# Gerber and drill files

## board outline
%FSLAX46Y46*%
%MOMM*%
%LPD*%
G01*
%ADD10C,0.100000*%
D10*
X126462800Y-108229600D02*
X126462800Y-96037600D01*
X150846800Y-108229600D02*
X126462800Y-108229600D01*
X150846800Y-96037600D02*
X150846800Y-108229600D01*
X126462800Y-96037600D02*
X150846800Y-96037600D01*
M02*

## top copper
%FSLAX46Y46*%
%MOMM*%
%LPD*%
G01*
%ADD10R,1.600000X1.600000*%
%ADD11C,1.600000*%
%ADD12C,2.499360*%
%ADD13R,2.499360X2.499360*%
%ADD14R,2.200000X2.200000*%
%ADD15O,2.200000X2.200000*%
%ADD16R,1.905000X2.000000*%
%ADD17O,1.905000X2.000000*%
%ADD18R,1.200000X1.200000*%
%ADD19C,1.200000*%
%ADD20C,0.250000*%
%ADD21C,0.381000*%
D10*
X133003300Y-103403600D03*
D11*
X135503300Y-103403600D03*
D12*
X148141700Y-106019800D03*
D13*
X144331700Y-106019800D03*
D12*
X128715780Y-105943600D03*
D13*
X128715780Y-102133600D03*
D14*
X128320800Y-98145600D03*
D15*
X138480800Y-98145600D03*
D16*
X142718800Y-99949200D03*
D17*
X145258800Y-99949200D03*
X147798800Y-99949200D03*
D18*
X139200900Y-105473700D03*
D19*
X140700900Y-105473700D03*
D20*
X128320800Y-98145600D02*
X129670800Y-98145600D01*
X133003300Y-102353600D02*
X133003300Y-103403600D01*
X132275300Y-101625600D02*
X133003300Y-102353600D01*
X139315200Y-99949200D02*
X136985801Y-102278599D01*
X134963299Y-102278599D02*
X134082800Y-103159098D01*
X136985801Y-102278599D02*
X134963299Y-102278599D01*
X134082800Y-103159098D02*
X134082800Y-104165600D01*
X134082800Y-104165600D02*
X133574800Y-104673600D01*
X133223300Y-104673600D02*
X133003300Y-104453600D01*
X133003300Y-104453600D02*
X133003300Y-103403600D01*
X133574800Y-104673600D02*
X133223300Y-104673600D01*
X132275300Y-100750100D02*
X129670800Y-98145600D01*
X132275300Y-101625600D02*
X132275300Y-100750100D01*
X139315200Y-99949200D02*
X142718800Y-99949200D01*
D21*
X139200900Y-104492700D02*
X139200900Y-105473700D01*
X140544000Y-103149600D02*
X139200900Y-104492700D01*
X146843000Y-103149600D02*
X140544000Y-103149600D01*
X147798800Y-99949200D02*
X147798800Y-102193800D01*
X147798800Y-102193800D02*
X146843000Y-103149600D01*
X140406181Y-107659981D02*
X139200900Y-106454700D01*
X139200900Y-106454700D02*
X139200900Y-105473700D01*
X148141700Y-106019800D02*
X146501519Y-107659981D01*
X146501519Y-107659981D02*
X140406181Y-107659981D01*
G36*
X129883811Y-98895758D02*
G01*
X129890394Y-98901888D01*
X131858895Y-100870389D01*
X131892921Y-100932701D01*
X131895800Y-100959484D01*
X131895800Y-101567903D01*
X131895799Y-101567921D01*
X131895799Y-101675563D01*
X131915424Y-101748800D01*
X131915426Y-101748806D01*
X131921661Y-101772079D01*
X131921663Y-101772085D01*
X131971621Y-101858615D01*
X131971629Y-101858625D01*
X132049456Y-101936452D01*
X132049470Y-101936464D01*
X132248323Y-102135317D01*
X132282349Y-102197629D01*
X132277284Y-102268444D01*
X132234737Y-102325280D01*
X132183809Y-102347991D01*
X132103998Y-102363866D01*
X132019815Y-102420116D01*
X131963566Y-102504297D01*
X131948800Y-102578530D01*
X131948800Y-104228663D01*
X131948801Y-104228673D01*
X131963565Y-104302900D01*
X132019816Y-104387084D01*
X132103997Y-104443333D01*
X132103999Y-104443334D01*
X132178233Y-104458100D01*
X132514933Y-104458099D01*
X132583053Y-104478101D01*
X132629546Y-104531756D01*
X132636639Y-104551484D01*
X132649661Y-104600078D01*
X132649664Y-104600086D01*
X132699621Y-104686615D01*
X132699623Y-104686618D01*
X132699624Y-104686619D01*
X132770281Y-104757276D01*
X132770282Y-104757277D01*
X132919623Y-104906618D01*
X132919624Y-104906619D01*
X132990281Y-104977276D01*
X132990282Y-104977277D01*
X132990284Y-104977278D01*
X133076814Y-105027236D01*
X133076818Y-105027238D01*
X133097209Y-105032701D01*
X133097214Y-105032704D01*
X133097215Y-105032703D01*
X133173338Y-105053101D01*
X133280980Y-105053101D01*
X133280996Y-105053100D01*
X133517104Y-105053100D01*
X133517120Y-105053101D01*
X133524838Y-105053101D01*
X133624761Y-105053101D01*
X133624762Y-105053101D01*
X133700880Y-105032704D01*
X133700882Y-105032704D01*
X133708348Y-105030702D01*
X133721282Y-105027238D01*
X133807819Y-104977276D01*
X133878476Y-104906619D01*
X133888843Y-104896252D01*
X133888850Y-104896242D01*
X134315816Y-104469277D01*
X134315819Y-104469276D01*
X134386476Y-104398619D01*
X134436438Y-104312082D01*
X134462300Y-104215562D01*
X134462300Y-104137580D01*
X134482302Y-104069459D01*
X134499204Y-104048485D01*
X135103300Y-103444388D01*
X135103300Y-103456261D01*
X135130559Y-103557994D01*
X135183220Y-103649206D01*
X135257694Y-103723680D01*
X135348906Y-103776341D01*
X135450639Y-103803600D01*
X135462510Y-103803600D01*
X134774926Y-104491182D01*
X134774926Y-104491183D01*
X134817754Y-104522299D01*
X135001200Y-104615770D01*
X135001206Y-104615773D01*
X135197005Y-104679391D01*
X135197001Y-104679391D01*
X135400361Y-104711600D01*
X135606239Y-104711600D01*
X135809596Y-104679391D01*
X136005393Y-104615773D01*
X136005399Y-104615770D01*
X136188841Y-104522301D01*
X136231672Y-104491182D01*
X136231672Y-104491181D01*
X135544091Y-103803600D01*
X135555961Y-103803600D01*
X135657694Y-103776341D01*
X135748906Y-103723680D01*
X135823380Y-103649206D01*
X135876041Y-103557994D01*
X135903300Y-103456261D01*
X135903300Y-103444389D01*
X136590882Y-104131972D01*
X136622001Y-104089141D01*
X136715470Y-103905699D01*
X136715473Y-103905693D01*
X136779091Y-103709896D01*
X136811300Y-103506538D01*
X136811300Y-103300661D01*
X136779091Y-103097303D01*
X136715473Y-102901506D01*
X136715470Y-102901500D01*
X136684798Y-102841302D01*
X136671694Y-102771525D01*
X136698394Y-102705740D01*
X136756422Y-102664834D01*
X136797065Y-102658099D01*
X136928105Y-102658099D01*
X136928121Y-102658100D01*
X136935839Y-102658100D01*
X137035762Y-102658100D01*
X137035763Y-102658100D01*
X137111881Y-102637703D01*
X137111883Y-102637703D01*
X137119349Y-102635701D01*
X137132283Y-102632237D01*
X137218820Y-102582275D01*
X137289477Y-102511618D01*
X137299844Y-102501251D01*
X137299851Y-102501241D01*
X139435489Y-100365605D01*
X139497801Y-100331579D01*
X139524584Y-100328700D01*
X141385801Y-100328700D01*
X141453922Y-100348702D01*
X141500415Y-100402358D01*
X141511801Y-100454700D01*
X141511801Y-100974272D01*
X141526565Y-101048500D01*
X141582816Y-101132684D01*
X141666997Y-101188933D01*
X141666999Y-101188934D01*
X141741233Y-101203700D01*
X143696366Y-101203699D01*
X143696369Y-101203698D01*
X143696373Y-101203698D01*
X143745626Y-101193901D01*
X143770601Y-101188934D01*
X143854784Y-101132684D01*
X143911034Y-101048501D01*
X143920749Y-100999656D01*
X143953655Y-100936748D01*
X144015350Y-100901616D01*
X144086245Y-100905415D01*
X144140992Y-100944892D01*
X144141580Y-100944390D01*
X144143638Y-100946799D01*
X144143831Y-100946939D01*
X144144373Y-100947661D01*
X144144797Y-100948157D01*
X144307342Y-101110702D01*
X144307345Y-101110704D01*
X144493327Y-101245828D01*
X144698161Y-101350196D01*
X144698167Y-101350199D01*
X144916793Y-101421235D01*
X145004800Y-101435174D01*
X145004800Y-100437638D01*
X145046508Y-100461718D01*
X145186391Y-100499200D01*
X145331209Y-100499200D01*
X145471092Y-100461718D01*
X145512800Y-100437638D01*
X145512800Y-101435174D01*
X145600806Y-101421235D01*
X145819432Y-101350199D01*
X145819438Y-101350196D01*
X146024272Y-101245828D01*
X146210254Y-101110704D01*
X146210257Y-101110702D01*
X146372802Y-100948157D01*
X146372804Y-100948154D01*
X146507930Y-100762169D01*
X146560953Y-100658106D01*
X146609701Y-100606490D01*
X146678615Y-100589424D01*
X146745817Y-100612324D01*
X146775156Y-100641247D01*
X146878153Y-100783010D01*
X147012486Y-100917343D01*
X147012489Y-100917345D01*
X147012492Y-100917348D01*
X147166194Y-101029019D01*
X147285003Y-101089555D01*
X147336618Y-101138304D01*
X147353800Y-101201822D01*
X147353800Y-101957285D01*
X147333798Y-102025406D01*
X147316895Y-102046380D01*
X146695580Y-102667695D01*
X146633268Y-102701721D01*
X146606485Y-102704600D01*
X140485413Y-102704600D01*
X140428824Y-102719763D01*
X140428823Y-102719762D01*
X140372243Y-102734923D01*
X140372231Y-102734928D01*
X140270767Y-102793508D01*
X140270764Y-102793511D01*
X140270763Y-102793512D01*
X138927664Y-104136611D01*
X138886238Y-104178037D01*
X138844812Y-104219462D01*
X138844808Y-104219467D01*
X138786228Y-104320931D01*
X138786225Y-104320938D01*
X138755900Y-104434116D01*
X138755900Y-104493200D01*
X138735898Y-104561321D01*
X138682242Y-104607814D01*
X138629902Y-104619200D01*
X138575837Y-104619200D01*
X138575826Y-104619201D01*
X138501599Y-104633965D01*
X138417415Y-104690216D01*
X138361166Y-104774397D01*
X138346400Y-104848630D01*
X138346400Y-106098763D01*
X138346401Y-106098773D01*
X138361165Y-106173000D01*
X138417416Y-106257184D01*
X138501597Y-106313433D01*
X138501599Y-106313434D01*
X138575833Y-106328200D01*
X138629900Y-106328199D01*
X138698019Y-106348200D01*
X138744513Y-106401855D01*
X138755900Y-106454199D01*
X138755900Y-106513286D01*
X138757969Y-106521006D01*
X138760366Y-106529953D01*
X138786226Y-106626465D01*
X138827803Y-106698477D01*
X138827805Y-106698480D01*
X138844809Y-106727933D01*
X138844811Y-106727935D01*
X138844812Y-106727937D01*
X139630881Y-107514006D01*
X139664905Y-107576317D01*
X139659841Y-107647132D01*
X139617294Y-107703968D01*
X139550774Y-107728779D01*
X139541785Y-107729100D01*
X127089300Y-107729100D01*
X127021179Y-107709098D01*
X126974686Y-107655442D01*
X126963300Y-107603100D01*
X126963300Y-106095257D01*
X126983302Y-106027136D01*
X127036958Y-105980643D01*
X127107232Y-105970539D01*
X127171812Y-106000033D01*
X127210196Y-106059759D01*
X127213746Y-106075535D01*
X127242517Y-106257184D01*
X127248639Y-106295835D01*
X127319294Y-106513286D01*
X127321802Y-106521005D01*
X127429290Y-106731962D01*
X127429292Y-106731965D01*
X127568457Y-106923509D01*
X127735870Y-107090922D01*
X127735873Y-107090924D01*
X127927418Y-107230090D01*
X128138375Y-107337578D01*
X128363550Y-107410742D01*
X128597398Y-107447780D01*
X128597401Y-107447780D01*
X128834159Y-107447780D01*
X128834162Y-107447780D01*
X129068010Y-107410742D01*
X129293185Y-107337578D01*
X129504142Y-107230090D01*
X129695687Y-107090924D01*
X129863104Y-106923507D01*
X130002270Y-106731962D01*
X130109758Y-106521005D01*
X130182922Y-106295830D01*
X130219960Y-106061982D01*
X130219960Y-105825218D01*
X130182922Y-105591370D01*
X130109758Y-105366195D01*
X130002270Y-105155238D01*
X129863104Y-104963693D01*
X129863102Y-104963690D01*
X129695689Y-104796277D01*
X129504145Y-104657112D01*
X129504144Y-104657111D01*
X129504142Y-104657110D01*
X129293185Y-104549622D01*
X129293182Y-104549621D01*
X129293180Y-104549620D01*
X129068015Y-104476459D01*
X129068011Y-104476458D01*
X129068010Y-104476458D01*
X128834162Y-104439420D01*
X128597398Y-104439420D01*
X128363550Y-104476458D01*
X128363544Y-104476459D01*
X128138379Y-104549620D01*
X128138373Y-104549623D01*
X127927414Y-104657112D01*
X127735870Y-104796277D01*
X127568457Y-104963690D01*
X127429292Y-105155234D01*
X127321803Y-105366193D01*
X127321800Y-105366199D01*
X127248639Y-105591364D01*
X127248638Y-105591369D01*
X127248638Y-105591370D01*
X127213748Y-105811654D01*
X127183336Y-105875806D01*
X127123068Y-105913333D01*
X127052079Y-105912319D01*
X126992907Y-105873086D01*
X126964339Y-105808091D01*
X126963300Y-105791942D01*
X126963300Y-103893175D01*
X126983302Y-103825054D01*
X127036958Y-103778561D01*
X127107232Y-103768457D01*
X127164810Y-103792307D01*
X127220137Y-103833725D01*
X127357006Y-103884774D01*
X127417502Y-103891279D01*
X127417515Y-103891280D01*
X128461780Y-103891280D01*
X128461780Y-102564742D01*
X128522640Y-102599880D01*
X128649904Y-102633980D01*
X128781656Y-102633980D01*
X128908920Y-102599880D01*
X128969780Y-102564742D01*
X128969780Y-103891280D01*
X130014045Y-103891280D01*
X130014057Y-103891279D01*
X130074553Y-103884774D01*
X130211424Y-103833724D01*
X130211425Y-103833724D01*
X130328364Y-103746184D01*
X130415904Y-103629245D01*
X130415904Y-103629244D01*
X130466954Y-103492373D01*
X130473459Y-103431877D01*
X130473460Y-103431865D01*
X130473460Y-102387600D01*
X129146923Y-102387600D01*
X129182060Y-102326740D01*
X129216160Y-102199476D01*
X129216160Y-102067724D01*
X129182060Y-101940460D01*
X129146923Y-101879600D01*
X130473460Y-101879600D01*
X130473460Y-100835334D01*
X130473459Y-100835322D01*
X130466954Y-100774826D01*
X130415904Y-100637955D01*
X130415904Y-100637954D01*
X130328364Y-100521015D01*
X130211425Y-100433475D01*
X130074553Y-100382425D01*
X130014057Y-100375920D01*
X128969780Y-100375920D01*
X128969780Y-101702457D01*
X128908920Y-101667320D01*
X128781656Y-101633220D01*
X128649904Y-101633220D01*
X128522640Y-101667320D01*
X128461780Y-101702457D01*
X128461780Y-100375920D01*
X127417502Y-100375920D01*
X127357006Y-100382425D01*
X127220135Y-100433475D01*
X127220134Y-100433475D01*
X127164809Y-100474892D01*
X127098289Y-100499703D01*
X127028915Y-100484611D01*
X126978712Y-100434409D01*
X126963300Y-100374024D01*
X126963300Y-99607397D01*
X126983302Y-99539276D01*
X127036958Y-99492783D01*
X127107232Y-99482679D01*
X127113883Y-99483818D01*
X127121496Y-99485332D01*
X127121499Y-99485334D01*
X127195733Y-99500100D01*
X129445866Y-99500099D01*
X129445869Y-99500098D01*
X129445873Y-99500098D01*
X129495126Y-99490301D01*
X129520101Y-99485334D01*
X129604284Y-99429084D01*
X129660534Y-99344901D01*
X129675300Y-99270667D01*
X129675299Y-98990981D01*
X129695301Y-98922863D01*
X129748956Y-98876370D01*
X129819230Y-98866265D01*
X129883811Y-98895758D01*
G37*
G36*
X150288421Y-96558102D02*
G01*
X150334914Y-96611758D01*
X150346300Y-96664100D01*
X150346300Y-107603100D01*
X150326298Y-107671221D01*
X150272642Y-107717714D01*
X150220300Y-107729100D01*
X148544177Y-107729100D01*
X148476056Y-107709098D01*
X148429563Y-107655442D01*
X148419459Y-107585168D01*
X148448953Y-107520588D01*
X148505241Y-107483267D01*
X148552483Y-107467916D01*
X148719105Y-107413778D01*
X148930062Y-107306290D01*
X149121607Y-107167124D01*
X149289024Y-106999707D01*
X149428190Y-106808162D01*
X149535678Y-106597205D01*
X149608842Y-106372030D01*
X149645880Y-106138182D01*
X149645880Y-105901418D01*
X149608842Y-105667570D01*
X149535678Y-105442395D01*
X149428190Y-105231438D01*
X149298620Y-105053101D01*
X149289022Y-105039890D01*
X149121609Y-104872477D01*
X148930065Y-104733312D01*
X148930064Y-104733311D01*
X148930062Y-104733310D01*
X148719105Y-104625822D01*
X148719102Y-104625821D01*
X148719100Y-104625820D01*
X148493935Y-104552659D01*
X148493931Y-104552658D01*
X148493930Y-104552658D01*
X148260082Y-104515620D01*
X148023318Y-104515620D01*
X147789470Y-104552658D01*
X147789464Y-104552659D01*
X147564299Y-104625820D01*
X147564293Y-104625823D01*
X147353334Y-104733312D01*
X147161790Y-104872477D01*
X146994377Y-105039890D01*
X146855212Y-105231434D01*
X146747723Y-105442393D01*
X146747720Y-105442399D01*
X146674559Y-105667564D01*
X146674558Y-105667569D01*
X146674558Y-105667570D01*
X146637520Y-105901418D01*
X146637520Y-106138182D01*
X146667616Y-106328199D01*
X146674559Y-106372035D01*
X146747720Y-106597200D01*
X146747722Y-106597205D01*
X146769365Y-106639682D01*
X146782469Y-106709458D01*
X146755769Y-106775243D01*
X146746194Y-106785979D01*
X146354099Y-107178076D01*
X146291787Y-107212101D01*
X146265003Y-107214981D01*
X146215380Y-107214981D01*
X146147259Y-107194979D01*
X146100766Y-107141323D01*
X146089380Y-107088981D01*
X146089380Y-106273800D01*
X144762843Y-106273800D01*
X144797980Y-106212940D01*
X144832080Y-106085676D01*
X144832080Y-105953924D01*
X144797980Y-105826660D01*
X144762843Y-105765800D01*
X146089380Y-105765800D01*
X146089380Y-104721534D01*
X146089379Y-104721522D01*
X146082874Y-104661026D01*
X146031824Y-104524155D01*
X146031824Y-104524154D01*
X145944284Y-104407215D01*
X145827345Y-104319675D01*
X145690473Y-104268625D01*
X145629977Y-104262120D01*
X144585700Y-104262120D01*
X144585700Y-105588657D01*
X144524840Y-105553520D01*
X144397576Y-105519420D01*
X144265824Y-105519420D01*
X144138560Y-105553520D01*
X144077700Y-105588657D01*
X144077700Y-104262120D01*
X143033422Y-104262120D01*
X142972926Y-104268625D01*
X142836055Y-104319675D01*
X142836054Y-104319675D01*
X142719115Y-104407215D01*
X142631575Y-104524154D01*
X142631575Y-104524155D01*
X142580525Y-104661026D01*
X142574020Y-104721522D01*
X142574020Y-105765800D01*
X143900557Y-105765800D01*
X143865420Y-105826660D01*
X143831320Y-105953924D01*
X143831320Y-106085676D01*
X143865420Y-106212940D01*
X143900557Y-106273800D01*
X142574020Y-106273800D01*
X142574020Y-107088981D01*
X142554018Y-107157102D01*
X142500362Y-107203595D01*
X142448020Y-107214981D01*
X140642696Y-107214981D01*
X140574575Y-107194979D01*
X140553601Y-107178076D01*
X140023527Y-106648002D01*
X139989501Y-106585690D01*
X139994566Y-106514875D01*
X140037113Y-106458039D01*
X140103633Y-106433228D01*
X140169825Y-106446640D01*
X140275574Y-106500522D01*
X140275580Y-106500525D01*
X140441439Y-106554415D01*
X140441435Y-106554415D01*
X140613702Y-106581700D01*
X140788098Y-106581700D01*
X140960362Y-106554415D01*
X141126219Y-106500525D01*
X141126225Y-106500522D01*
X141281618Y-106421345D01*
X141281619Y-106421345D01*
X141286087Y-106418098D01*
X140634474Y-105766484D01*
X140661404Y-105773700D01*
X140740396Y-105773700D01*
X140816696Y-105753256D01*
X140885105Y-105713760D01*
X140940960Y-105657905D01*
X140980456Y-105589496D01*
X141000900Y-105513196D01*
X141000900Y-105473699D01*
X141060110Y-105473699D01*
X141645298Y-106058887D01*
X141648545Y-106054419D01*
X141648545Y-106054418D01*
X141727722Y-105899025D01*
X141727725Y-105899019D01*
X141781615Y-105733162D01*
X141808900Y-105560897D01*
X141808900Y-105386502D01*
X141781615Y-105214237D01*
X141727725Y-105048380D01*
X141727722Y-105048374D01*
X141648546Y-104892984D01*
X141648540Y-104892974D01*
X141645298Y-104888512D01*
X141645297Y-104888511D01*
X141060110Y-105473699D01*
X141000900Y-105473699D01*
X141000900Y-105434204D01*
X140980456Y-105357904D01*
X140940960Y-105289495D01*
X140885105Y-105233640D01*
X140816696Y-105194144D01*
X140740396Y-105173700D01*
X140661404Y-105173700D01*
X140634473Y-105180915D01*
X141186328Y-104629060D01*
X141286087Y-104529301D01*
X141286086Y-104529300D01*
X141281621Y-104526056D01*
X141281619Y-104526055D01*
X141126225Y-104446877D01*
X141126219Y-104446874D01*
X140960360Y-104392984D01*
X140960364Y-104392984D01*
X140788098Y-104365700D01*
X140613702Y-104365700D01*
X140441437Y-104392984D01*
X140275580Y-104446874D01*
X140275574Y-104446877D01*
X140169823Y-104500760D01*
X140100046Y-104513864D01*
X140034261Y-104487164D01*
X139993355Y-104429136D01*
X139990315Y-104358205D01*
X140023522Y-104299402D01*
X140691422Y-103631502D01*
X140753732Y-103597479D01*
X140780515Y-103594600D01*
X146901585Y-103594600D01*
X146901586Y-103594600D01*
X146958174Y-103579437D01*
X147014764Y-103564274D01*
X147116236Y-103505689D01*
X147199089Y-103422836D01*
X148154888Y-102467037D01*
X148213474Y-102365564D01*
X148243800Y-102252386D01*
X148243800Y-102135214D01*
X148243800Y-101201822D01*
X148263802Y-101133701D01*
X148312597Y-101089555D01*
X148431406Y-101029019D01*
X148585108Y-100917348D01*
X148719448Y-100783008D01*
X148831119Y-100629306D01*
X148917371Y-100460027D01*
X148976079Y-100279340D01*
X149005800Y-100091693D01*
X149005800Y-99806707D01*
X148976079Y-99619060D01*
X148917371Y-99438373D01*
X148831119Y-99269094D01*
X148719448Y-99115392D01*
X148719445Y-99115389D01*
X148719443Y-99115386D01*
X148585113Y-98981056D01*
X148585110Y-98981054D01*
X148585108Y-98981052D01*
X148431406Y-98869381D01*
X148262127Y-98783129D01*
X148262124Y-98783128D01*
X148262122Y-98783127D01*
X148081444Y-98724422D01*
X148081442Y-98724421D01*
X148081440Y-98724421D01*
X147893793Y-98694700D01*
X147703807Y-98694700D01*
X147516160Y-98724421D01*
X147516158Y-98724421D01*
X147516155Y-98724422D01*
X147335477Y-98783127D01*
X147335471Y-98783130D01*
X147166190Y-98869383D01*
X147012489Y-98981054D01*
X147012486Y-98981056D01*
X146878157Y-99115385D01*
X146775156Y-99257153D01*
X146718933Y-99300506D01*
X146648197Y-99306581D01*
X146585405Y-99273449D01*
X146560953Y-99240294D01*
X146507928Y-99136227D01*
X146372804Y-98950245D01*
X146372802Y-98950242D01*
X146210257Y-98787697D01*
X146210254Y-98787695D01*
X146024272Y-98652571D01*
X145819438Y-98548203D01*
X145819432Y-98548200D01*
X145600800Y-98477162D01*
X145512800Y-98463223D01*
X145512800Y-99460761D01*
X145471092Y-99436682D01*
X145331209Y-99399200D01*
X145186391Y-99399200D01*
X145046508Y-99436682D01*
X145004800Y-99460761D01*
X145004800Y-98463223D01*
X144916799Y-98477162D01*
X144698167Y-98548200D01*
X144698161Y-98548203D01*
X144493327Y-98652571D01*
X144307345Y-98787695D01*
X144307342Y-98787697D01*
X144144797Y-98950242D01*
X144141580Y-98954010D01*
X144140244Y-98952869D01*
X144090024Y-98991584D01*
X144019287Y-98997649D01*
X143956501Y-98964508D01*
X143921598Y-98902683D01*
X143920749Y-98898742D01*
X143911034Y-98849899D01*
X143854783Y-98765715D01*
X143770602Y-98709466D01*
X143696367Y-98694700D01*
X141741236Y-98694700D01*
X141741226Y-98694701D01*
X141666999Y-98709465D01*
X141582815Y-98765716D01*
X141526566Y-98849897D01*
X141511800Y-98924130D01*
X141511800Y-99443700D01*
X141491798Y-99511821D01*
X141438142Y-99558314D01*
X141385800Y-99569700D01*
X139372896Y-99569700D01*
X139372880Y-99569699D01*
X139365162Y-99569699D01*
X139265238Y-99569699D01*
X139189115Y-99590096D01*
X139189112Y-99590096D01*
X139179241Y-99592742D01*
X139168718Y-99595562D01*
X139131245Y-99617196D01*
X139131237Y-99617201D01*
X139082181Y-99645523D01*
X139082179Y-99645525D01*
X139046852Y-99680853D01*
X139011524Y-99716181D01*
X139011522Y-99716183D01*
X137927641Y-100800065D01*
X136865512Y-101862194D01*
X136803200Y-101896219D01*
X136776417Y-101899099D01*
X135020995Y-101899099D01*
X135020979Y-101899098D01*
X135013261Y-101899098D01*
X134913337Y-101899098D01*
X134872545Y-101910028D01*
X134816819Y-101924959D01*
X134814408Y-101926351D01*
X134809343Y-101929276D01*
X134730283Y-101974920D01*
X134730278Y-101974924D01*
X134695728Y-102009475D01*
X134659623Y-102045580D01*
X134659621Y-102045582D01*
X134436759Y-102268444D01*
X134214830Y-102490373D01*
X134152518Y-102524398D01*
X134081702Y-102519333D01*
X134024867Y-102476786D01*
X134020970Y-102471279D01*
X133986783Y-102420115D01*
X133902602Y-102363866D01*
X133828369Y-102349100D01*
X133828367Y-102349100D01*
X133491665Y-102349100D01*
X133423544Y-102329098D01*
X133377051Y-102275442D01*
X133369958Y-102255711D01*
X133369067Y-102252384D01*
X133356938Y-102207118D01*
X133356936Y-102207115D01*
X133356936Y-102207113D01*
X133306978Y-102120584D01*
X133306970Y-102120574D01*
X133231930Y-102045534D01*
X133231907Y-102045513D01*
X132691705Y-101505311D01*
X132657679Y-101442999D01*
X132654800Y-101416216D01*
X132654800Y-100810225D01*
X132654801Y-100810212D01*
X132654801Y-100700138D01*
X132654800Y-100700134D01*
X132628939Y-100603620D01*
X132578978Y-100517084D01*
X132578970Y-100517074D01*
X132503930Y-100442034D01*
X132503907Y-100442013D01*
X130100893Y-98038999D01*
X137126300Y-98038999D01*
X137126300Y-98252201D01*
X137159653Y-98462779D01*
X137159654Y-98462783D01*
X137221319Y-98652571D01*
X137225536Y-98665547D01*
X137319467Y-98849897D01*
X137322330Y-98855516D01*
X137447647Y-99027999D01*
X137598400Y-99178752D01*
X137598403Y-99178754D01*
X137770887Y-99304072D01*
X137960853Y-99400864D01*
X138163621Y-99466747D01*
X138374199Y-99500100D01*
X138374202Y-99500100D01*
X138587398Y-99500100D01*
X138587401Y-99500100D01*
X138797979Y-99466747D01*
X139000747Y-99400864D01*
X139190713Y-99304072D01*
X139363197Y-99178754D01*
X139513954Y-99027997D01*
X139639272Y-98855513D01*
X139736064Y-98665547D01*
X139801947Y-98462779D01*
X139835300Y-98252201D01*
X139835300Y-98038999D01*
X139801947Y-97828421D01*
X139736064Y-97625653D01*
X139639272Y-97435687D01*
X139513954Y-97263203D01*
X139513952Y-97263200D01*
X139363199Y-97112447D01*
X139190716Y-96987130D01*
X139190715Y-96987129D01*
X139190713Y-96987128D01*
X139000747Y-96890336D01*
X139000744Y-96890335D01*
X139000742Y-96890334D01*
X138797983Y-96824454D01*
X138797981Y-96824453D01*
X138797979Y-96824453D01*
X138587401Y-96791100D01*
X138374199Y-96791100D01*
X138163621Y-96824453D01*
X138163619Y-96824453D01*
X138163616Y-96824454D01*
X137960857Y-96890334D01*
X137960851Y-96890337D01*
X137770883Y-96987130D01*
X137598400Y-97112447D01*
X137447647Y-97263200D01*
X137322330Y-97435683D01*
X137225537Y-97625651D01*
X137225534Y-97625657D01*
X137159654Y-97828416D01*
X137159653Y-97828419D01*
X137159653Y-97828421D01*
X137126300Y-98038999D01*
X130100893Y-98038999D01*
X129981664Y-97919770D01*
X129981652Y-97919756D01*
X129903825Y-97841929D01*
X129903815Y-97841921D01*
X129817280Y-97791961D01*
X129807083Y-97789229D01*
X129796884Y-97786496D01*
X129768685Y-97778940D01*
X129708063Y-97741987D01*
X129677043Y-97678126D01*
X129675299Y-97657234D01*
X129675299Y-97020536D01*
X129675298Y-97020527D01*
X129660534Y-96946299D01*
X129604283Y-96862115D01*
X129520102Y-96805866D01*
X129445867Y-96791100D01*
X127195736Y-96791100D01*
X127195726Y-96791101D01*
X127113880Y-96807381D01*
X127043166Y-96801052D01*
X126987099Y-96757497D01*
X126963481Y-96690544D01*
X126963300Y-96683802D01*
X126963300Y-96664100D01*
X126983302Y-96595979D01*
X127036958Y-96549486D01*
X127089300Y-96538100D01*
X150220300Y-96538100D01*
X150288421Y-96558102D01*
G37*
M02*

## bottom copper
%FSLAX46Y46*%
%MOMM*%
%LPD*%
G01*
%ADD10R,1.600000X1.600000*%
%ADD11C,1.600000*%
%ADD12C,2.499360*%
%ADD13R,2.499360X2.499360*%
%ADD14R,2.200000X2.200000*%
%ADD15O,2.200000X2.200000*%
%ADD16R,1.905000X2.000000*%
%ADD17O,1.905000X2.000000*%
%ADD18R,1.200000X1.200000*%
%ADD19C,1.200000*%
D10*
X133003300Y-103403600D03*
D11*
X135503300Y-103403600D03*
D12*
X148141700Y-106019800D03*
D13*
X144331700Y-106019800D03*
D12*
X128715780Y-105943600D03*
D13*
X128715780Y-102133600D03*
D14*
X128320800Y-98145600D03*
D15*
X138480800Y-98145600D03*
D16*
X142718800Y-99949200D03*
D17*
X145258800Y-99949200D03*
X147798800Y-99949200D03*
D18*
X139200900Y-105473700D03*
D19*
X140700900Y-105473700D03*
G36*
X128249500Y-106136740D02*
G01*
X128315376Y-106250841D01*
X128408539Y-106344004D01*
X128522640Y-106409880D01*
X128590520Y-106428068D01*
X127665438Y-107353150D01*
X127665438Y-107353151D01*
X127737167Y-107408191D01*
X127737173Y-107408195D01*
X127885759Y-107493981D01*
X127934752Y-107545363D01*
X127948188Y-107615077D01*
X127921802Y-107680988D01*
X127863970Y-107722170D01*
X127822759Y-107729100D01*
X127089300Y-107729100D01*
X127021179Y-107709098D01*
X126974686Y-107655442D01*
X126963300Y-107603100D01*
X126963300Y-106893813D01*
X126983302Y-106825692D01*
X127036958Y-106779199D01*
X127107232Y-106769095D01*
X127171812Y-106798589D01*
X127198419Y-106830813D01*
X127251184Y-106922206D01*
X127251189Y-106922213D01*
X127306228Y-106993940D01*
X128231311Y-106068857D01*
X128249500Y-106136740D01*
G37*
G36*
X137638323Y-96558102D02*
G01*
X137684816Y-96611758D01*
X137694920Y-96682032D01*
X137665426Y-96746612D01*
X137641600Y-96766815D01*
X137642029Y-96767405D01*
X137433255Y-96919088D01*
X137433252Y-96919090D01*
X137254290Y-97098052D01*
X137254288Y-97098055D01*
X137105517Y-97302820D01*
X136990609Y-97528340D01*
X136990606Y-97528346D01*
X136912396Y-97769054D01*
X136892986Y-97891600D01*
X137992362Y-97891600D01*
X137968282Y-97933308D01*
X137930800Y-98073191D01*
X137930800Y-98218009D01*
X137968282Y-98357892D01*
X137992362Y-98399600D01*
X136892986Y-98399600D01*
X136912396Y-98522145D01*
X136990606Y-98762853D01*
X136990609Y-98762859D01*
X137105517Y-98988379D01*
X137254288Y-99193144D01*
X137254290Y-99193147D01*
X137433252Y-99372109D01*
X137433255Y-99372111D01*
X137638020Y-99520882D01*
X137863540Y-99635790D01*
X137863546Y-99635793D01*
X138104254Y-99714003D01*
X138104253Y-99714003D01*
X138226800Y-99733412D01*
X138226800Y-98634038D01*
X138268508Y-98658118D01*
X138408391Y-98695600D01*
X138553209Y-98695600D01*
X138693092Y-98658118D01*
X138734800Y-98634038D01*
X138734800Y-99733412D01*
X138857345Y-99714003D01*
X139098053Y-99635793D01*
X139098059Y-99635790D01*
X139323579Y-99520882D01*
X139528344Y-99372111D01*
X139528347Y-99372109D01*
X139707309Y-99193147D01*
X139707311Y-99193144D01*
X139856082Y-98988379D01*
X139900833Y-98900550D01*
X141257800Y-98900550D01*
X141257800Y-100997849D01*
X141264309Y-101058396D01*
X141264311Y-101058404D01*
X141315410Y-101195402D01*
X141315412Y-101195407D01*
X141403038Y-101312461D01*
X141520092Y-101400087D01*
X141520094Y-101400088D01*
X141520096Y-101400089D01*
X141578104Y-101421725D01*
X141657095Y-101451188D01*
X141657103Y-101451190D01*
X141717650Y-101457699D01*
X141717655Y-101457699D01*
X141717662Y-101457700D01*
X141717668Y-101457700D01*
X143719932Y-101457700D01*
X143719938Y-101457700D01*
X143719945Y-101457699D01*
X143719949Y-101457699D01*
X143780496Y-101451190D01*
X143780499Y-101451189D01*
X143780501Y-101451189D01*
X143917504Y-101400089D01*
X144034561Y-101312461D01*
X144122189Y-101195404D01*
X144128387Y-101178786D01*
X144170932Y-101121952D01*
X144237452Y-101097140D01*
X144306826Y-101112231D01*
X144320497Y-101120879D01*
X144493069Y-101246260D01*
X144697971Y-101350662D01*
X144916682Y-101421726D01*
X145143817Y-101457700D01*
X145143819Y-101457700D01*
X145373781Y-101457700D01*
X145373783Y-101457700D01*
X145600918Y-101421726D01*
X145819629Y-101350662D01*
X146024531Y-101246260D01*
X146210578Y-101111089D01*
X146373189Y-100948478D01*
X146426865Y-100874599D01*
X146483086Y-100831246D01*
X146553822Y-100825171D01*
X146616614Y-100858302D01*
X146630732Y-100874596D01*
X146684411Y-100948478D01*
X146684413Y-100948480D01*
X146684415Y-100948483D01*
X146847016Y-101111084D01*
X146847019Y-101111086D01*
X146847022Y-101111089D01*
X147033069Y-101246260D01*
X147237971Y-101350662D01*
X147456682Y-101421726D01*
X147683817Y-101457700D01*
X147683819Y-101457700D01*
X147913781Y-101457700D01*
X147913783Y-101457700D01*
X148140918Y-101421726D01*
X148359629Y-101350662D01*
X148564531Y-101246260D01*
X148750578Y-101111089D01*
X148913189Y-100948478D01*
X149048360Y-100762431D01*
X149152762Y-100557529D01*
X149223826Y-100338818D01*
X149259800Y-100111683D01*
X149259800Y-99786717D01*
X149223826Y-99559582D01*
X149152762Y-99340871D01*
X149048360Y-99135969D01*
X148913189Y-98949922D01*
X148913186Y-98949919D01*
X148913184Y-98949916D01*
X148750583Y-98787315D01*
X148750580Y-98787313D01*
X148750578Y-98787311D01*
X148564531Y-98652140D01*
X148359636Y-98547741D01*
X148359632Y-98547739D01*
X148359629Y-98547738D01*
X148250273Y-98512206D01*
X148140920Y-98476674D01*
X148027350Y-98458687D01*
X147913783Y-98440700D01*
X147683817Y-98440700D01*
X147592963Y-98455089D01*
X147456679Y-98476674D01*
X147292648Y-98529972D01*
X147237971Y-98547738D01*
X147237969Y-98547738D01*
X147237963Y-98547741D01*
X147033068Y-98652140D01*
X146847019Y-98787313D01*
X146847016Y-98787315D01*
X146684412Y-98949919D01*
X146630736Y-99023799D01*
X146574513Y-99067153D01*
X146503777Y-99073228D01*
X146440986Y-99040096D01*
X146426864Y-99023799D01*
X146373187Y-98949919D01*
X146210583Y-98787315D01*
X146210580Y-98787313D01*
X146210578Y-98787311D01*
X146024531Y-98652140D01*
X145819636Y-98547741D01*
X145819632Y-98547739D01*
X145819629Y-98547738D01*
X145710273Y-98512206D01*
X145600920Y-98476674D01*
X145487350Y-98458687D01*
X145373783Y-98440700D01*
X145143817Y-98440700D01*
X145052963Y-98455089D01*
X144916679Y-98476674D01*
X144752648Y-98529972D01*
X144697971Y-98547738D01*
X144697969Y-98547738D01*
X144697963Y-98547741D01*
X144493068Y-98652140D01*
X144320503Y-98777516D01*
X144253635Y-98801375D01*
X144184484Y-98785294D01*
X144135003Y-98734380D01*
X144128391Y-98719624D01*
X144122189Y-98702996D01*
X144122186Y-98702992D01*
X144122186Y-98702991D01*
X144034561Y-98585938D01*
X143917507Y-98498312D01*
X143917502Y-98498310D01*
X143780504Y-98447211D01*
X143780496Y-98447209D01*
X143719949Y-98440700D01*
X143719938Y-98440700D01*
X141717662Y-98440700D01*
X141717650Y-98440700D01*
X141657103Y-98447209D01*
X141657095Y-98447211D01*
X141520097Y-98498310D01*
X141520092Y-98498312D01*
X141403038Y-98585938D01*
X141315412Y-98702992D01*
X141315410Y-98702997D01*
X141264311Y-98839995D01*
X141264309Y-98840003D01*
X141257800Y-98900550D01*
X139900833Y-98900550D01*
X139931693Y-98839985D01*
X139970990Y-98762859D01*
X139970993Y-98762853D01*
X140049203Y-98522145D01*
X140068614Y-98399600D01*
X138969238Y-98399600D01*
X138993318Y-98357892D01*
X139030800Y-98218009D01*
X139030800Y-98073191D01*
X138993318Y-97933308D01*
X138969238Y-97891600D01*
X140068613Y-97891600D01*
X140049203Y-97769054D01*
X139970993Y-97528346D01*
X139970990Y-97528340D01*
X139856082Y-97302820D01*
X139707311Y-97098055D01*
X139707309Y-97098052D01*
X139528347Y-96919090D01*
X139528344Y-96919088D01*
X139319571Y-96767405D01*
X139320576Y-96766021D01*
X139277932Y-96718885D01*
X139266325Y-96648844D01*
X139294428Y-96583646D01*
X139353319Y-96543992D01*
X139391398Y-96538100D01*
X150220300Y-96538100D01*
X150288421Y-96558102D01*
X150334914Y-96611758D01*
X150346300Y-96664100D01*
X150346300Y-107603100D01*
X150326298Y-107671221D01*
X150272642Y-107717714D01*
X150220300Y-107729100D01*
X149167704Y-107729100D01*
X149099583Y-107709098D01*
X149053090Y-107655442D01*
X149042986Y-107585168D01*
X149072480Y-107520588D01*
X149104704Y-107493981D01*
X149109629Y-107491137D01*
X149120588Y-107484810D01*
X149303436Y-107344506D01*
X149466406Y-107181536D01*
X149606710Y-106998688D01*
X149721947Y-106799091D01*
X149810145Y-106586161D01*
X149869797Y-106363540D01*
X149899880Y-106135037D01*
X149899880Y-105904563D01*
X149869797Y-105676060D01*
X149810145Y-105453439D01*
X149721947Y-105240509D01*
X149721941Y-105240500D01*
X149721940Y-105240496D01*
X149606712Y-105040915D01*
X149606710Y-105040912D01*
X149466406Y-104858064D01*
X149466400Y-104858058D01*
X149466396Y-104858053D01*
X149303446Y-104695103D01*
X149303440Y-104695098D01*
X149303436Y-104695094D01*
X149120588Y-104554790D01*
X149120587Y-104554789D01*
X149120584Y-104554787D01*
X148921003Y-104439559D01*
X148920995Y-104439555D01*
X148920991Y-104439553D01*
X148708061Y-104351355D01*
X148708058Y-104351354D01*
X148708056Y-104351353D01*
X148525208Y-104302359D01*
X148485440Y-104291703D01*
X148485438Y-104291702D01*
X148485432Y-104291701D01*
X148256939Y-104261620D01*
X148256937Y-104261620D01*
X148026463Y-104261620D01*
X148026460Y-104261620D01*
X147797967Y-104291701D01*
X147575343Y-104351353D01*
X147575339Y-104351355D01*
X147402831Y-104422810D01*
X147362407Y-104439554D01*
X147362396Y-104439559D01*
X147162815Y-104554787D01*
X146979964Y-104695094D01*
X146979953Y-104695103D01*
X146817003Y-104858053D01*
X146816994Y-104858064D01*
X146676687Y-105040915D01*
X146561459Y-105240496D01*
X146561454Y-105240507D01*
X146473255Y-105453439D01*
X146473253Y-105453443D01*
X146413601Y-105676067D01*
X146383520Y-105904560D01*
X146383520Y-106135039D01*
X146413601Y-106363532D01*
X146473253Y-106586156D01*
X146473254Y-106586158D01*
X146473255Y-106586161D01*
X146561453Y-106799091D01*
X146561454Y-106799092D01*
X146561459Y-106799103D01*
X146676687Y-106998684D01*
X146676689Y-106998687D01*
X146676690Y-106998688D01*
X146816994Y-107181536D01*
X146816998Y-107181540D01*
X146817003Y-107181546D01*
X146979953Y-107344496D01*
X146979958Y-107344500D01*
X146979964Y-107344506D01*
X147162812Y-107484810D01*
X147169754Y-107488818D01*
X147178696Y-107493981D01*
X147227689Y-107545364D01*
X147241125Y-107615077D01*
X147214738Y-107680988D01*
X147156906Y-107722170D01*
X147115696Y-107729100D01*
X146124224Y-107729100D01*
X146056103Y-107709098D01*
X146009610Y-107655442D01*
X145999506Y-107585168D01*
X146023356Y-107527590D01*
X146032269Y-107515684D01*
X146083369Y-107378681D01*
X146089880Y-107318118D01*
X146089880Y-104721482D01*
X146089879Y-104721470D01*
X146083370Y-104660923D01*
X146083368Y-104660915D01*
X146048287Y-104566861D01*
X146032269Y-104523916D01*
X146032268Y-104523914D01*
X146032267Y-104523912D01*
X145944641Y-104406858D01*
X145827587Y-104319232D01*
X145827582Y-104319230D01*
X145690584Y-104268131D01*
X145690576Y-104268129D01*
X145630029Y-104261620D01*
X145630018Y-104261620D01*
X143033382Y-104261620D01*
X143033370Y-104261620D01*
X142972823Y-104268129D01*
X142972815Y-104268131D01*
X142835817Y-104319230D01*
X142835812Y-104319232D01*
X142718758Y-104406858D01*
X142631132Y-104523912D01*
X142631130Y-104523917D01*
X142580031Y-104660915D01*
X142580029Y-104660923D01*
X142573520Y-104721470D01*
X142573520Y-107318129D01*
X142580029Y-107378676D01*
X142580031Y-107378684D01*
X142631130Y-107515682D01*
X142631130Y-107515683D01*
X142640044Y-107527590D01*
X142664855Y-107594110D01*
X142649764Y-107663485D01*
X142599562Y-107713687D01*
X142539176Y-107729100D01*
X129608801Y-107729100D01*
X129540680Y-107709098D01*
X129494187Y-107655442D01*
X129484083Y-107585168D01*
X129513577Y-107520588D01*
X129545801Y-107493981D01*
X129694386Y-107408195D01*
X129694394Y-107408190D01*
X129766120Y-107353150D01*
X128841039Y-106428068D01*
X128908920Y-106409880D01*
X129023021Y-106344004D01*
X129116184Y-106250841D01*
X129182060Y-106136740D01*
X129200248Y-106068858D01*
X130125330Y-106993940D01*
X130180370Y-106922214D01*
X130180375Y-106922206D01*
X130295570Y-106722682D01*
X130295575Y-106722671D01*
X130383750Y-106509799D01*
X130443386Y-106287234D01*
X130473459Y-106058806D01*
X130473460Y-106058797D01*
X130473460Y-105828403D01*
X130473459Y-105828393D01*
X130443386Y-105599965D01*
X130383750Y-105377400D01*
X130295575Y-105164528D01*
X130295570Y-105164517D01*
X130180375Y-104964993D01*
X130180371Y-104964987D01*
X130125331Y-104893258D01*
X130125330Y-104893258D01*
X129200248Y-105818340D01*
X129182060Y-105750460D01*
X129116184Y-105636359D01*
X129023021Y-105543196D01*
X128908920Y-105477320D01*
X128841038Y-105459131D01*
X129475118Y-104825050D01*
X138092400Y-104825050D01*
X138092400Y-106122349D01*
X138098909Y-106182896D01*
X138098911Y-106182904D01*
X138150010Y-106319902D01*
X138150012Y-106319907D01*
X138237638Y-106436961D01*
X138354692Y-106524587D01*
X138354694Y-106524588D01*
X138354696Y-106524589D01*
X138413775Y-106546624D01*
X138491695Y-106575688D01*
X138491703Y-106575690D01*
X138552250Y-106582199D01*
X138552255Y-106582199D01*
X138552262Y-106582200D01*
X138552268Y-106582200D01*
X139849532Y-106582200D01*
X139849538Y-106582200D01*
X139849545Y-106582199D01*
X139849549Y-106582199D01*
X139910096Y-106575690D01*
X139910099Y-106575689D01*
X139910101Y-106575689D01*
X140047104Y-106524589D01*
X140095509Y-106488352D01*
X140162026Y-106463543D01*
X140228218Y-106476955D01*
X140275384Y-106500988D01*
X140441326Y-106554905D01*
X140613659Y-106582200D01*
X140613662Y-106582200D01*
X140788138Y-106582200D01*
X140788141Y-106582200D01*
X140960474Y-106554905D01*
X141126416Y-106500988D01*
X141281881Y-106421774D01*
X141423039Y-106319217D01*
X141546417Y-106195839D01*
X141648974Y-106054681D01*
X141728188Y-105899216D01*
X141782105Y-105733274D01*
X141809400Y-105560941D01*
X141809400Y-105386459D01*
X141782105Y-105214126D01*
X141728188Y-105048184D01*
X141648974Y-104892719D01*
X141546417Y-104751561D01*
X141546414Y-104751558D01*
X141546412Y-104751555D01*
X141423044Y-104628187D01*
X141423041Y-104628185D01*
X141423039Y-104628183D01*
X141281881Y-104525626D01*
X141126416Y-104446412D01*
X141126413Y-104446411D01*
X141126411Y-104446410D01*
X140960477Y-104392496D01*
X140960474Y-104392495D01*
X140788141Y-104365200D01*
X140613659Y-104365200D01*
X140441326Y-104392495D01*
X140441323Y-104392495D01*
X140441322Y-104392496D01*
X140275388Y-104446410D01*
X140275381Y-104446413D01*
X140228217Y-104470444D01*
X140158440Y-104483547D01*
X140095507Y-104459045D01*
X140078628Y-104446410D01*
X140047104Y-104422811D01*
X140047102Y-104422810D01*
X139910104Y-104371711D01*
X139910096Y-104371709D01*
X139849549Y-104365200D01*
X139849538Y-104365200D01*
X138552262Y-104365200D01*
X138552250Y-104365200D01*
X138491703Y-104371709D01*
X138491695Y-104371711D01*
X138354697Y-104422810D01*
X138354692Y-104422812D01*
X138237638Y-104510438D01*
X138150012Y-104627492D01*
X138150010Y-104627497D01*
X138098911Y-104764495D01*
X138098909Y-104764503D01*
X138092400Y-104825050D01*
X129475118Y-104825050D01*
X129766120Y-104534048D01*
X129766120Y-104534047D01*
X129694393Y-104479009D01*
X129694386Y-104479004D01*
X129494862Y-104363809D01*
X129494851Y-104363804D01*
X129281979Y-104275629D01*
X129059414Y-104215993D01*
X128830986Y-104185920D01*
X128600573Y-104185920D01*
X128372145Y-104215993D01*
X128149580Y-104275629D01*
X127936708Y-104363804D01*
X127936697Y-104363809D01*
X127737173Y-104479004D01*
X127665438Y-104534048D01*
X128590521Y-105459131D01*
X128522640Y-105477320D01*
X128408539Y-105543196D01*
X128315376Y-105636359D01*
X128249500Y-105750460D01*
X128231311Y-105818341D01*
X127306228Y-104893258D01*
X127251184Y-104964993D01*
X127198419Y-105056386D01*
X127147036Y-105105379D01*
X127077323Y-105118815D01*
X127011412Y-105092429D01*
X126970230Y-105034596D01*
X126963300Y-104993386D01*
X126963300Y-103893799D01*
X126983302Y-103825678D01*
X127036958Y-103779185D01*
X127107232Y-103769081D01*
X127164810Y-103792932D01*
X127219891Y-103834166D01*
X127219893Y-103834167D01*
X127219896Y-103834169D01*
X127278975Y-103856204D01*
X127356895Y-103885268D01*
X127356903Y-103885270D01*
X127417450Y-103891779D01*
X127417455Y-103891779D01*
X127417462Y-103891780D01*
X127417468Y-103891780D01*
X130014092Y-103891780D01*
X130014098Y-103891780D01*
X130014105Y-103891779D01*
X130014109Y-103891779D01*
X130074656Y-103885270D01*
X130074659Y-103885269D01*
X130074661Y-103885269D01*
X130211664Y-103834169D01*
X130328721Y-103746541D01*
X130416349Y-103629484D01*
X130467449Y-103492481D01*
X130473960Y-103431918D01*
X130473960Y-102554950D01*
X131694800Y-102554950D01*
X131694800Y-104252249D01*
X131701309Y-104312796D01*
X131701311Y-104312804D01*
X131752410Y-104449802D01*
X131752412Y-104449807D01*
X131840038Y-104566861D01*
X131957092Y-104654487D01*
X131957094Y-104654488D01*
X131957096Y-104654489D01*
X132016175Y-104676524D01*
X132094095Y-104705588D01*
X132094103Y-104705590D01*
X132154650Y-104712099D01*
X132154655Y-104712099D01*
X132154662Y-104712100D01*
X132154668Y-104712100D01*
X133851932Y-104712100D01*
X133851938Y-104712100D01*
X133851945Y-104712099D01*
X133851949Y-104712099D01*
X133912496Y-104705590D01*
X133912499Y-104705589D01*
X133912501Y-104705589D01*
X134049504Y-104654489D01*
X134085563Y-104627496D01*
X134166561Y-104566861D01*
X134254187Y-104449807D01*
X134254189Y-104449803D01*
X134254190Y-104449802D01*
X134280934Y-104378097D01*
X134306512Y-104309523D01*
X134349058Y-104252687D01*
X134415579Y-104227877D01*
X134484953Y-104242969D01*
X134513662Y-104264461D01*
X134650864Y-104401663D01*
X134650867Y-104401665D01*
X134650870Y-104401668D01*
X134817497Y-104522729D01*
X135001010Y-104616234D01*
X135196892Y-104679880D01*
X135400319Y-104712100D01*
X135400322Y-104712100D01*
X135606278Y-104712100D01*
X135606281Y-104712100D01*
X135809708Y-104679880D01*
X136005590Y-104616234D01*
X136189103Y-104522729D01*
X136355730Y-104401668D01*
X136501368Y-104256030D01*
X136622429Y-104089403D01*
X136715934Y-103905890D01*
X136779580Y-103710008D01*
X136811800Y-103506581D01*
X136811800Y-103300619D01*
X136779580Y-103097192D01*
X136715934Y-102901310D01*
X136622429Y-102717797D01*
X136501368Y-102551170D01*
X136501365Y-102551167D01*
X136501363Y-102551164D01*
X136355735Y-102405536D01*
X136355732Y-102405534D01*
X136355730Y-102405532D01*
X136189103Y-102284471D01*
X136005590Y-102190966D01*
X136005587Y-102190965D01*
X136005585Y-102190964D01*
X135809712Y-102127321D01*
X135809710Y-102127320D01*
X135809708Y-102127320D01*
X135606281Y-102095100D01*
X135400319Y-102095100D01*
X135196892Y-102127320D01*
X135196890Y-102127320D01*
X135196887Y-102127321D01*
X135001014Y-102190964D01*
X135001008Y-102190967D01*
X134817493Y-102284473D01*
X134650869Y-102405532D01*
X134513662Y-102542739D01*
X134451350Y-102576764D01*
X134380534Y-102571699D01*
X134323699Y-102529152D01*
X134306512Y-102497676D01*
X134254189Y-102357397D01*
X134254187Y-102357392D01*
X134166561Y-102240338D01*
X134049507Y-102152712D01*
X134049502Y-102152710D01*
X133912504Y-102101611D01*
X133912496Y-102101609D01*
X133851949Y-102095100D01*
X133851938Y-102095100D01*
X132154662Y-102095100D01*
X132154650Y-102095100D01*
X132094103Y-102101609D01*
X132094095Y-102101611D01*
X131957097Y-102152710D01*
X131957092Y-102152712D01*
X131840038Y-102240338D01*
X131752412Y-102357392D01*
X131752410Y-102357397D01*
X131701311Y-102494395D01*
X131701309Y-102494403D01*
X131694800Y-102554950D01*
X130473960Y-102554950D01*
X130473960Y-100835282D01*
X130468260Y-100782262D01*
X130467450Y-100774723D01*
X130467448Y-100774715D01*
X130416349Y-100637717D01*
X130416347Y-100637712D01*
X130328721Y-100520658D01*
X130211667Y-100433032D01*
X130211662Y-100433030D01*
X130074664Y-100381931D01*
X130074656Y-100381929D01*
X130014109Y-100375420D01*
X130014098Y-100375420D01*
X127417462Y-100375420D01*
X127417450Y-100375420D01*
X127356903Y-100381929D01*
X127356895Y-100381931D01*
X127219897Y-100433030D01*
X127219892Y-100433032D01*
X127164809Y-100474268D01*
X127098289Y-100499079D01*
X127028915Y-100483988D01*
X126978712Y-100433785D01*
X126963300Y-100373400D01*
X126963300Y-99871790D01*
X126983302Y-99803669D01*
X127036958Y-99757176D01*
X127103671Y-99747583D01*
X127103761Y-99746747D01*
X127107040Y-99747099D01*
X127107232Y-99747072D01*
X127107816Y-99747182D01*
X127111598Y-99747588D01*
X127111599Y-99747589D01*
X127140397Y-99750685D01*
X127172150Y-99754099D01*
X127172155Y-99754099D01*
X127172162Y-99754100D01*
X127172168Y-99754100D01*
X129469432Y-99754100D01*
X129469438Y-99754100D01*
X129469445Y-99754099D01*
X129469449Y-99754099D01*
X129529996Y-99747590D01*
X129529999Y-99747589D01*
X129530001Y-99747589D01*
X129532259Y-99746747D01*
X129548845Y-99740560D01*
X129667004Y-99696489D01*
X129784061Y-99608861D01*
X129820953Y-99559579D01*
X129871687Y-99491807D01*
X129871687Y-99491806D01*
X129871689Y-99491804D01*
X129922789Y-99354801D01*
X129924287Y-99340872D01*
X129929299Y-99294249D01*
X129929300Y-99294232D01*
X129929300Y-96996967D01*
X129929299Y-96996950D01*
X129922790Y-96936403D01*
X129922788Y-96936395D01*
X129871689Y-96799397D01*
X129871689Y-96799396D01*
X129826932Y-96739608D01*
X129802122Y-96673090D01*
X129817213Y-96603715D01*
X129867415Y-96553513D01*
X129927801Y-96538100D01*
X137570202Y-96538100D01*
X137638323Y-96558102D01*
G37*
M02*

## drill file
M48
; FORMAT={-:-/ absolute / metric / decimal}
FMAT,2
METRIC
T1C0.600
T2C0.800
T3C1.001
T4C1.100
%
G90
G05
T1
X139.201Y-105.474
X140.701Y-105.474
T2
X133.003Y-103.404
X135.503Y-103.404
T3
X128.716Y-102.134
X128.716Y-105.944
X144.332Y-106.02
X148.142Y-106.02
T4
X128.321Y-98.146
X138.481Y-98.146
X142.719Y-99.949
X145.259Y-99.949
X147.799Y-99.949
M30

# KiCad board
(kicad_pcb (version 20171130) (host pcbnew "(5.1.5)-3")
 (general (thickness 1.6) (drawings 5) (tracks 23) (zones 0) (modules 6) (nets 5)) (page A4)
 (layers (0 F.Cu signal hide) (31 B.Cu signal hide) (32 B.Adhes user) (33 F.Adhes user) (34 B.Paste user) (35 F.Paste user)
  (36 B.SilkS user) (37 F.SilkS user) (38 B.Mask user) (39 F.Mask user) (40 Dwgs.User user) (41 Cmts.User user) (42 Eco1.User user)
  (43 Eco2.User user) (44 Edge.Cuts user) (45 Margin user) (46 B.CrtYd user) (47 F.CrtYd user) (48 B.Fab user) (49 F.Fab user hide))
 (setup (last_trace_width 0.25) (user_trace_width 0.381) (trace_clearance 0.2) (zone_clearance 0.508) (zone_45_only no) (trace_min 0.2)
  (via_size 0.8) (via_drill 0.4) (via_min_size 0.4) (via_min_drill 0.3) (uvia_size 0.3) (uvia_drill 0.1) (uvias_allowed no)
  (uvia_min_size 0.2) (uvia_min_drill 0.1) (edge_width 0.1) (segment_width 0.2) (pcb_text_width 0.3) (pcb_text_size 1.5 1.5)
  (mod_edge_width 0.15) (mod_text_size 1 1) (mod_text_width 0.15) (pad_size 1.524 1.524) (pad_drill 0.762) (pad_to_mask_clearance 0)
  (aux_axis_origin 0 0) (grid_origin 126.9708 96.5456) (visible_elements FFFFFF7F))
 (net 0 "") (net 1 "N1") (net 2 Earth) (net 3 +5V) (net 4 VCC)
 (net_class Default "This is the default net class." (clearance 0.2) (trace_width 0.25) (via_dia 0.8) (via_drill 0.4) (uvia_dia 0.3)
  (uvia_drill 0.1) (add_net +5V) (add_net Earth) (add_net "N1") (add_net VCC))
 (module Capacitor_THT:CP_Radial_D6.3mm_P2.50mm (layer F.Cu) (at 133.0033 103.4036)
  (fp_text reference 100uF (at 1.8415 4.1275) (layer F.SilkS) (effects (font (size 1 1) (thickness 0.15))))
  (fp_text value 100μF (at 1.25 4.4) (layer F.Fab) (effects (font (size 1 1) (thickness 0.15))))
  (pad 1 thru_hole rect (at 0 0) (size 1.6 1.6) (drill 0.8) (layers *.Cu *.Mask) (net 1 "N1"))
  (pad 2 thru_hole circle (at 2.5 0) (size 1.6 1.6) (drill 0.8) (layers *.Cu *.Mask) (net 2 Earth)))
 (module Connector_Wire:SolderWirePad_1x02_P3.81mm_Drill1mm (layer F.Cu) (at 144.3317 106.0198)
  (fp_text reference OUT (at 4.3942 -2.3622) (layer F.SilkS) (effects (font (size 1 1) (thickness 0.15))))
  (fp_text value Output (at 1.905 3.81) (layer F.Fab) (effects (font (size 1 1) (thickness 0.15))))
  (pad 2 thru_hole circle (at 3.81 0) (size 2.49936 2.49936) (drill 1.00076) (layers *.Cu *.Mask) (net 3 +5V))
  (pad 1 thru_hole rect (at 0 0) (size 2.49936 2.49936) (drill 1.00076) (layers *.Cu *.Mask) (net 2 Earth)))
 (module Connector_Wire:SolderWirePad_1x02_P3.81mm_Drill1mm (layer F.Cu) (at 128.71578 102.1336 270)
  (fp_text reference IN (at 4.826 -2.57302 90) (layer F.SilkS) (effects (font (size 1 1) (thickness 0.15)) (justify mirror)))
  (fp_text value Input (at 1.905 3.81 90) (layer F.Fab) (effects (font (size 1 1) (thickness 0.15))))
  (pad 2 thru_hole circle (at 3.81 0 270) (size 2.49936 2.49936) (drill 1.00076) (layers *.Cu *.Mask) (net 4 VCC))
  (pad 1 thru_hole rect (at 0 0 270) (size 2.49936 2.49936) (drill 1.00076) (layers *.Cu *.Mask) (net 2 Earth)))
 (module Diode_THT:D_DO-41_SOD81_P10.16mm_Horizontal (layer F.Cu) (at 128.3208 98.1456)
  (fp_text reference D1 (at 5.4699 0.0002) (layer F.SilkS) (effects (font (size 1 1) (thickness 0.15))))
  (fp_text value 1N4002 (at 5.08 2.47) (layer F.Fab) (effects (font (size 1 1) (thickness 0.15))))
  (pad 1 thru_hole rect (at 0 0) (size 2.2 2.2) (drill 1.1) (layers *.Cu *.Mask) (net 1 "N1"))
  (pad 2 thru_hole oval (at 10.16 0) (size 2.2 2.2) (drill 1.1) (layers *.Cu *.Mask) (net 4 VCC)))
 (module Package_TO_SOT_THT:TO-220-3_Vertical (layer F.Cu) (at 142.7188 99.9492)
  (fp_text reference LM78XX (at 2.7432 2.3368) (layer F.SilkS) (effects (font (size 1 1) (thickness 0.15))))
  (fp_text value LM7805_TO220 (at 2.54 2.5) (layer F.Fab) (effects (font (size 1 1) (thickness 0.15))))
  (pad 1 thru_hole rect (at 0 0) (size 1.905 2) (drill 1.1) (layers *.Cu *.Mask) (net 1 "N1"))
  (pad 2 thru_hole oval (at 2.54 0) (size 1.905 2) (drill 1.1) (layers *.Cu *.Mask) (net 2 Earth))
  (pad 3 thru_hole oval (at 5.08 0) (size 1.905 2) (drill 1.1) (layers *.Cu *.Mask) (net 3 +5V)))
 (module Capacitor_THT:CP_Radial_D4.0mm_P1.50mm (layer F.Cu) (at 139.2009 105.4737)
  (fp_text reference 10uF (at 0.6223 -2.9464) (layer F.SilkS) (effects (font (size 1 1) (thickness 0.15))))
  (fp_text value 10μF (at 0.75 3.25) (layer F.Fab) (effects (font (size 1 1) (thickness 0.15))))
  (pad 1 thru_hole rect (at 0 0) (size 1.2 1.2) (drill 0.6) (layers *.Cu *.Mask) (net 3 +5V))
  (pad 2 thru_hole circle (at 1.5 0) (size 1.2 1.2) (drill 0.6) (layers *.Cu *.Mask) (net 2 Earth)))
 (gr_line (start 126.4628 108.2296) (end 126.4628 96.0376) (layer Edge.Cuts) (width 0.1))
 (gr_line (start 150.8468 108.2296) (end 126.4628 108.2296) (layer Edge.Cuts) (width 0.1))
 (gr_line (start 150.8468 96.0376) (end 150.8468 108.2296) (layer Edge.Cuts) (width 0.1))
 (gr_line (start 126.4628 96.0376) (end 150.8468 96.0376) (layer Edge.Cuts) (width 0.1))
 (segment (start 128.3208 98.1456) (end 129.6708 98.1456) (width 0.25) (layer F.Cu) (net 1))
 (segment (start 133.0033 102.3536) (end 133.0033 103.4036) (width 0.25) (layer F.Cu) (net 1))
 (segment (start 132.2753 101.6256) (end 133.0033 102.3536) (width 0.25) (layer F.Cu) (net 1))
 (segment (start 139.3152 99.9492) (end 136.985801 102.278599) (width 0.25) (layer F.Cu) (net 1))
 (segment (start 134.963299 102.278599) (end 134.0828 103.159098) (width 0.25) (layer F.Cu) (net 1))
 (segment (start 136.985801 102.278599) (end 134.963299 102.278599) (width 0.25) (layer F.Cu) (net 1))
 (segment (start 134.0828 103.159098) (end 134.0828 104.1656) (width 0.25) (layer F.Cu) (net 1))
 (segment (start 134.0828 104.1656) (end 133.5748 104.6736) (width 0.25) (layer F.Cu) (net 1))
 (segment (start 133.2233 104.6736) (end 133.0033 104.4536) (width 0.25) (layer F.Cu) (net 1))
 (segment (start 133.0033 104.4536) (end 133.0033 103.4036) (width 0.25) (layer F.Cu) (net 1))
 (segment (start 133.5748 104.6736) (end 133.2233 104.6736) (width 0.25) (layer F.Cu) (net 1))
 (segment (start 132.2753 100.7501) (end 129.6708 98.1456) (width 0.25) (layer F.Cu) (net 1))
 (segment (start 132.2753 101.6256) (end 132.2753 100.7501) (width 0.25) (layer F.Cu) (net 1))
 (segment (start 139.3152 99.9492) (end 142.7188 99.9492) (width 0.25) (layer F.Cu) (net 1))
 (segment (start 139.2009 104.4927) (end 139.2009 105.4737) (width 0.381) (layer F.Cu) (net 3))
 (segment (start 140.544 103.1496) (end 139.2009 104.4927) (width 0.381) (layer F.Cu) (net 3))
 (segment (start 146.843 103.1496) (end 140.544 103.1496) (width 0.381) (layer F.Cu) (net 3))
 (segment (start 147.7988 99.9492) (end 147.7988 102.1938) (width 0.381) (layer F.Cu) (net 3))
 (segment (start 147.7988 102.1938) (end 146.843 103.1496) (width 0.381) (layer F.Cu) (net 3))
 (segment (start 140.406181 107.659981) (end 139.2009 106.4547) (width 0.381) (layer F.Cu) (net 3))
 (segment (start 139.2009 106.4547) (end 139.2009 105.4737) (width 0.381) (layer F.Cu) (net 3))
 (segment (start 148.1417 106.0198) (end 146.501519 107.659981) (width 0.381) (layer F.Cu) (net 3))
 (segment (start 146.501519 107.659981) (end 140.406181 107.659981) (width 0.381) (layer F.Cu) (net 3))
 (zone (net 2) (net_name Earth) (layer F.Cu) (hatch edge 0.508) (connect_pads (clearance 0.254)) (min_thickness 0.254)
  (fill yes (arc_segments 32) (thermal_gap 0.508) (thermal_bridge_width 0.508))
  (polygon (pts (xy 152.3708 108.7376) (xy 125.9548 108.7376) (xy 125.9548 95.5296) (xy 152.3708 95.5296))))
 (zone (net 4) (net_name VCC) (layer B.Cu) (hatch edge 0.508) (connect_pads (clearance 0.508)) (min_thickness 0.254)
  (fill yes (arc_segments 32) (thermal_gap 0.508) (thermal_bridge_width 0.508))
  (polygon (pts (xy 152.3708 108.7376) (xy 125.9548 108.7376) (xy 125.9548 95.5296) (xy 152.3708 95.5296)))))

